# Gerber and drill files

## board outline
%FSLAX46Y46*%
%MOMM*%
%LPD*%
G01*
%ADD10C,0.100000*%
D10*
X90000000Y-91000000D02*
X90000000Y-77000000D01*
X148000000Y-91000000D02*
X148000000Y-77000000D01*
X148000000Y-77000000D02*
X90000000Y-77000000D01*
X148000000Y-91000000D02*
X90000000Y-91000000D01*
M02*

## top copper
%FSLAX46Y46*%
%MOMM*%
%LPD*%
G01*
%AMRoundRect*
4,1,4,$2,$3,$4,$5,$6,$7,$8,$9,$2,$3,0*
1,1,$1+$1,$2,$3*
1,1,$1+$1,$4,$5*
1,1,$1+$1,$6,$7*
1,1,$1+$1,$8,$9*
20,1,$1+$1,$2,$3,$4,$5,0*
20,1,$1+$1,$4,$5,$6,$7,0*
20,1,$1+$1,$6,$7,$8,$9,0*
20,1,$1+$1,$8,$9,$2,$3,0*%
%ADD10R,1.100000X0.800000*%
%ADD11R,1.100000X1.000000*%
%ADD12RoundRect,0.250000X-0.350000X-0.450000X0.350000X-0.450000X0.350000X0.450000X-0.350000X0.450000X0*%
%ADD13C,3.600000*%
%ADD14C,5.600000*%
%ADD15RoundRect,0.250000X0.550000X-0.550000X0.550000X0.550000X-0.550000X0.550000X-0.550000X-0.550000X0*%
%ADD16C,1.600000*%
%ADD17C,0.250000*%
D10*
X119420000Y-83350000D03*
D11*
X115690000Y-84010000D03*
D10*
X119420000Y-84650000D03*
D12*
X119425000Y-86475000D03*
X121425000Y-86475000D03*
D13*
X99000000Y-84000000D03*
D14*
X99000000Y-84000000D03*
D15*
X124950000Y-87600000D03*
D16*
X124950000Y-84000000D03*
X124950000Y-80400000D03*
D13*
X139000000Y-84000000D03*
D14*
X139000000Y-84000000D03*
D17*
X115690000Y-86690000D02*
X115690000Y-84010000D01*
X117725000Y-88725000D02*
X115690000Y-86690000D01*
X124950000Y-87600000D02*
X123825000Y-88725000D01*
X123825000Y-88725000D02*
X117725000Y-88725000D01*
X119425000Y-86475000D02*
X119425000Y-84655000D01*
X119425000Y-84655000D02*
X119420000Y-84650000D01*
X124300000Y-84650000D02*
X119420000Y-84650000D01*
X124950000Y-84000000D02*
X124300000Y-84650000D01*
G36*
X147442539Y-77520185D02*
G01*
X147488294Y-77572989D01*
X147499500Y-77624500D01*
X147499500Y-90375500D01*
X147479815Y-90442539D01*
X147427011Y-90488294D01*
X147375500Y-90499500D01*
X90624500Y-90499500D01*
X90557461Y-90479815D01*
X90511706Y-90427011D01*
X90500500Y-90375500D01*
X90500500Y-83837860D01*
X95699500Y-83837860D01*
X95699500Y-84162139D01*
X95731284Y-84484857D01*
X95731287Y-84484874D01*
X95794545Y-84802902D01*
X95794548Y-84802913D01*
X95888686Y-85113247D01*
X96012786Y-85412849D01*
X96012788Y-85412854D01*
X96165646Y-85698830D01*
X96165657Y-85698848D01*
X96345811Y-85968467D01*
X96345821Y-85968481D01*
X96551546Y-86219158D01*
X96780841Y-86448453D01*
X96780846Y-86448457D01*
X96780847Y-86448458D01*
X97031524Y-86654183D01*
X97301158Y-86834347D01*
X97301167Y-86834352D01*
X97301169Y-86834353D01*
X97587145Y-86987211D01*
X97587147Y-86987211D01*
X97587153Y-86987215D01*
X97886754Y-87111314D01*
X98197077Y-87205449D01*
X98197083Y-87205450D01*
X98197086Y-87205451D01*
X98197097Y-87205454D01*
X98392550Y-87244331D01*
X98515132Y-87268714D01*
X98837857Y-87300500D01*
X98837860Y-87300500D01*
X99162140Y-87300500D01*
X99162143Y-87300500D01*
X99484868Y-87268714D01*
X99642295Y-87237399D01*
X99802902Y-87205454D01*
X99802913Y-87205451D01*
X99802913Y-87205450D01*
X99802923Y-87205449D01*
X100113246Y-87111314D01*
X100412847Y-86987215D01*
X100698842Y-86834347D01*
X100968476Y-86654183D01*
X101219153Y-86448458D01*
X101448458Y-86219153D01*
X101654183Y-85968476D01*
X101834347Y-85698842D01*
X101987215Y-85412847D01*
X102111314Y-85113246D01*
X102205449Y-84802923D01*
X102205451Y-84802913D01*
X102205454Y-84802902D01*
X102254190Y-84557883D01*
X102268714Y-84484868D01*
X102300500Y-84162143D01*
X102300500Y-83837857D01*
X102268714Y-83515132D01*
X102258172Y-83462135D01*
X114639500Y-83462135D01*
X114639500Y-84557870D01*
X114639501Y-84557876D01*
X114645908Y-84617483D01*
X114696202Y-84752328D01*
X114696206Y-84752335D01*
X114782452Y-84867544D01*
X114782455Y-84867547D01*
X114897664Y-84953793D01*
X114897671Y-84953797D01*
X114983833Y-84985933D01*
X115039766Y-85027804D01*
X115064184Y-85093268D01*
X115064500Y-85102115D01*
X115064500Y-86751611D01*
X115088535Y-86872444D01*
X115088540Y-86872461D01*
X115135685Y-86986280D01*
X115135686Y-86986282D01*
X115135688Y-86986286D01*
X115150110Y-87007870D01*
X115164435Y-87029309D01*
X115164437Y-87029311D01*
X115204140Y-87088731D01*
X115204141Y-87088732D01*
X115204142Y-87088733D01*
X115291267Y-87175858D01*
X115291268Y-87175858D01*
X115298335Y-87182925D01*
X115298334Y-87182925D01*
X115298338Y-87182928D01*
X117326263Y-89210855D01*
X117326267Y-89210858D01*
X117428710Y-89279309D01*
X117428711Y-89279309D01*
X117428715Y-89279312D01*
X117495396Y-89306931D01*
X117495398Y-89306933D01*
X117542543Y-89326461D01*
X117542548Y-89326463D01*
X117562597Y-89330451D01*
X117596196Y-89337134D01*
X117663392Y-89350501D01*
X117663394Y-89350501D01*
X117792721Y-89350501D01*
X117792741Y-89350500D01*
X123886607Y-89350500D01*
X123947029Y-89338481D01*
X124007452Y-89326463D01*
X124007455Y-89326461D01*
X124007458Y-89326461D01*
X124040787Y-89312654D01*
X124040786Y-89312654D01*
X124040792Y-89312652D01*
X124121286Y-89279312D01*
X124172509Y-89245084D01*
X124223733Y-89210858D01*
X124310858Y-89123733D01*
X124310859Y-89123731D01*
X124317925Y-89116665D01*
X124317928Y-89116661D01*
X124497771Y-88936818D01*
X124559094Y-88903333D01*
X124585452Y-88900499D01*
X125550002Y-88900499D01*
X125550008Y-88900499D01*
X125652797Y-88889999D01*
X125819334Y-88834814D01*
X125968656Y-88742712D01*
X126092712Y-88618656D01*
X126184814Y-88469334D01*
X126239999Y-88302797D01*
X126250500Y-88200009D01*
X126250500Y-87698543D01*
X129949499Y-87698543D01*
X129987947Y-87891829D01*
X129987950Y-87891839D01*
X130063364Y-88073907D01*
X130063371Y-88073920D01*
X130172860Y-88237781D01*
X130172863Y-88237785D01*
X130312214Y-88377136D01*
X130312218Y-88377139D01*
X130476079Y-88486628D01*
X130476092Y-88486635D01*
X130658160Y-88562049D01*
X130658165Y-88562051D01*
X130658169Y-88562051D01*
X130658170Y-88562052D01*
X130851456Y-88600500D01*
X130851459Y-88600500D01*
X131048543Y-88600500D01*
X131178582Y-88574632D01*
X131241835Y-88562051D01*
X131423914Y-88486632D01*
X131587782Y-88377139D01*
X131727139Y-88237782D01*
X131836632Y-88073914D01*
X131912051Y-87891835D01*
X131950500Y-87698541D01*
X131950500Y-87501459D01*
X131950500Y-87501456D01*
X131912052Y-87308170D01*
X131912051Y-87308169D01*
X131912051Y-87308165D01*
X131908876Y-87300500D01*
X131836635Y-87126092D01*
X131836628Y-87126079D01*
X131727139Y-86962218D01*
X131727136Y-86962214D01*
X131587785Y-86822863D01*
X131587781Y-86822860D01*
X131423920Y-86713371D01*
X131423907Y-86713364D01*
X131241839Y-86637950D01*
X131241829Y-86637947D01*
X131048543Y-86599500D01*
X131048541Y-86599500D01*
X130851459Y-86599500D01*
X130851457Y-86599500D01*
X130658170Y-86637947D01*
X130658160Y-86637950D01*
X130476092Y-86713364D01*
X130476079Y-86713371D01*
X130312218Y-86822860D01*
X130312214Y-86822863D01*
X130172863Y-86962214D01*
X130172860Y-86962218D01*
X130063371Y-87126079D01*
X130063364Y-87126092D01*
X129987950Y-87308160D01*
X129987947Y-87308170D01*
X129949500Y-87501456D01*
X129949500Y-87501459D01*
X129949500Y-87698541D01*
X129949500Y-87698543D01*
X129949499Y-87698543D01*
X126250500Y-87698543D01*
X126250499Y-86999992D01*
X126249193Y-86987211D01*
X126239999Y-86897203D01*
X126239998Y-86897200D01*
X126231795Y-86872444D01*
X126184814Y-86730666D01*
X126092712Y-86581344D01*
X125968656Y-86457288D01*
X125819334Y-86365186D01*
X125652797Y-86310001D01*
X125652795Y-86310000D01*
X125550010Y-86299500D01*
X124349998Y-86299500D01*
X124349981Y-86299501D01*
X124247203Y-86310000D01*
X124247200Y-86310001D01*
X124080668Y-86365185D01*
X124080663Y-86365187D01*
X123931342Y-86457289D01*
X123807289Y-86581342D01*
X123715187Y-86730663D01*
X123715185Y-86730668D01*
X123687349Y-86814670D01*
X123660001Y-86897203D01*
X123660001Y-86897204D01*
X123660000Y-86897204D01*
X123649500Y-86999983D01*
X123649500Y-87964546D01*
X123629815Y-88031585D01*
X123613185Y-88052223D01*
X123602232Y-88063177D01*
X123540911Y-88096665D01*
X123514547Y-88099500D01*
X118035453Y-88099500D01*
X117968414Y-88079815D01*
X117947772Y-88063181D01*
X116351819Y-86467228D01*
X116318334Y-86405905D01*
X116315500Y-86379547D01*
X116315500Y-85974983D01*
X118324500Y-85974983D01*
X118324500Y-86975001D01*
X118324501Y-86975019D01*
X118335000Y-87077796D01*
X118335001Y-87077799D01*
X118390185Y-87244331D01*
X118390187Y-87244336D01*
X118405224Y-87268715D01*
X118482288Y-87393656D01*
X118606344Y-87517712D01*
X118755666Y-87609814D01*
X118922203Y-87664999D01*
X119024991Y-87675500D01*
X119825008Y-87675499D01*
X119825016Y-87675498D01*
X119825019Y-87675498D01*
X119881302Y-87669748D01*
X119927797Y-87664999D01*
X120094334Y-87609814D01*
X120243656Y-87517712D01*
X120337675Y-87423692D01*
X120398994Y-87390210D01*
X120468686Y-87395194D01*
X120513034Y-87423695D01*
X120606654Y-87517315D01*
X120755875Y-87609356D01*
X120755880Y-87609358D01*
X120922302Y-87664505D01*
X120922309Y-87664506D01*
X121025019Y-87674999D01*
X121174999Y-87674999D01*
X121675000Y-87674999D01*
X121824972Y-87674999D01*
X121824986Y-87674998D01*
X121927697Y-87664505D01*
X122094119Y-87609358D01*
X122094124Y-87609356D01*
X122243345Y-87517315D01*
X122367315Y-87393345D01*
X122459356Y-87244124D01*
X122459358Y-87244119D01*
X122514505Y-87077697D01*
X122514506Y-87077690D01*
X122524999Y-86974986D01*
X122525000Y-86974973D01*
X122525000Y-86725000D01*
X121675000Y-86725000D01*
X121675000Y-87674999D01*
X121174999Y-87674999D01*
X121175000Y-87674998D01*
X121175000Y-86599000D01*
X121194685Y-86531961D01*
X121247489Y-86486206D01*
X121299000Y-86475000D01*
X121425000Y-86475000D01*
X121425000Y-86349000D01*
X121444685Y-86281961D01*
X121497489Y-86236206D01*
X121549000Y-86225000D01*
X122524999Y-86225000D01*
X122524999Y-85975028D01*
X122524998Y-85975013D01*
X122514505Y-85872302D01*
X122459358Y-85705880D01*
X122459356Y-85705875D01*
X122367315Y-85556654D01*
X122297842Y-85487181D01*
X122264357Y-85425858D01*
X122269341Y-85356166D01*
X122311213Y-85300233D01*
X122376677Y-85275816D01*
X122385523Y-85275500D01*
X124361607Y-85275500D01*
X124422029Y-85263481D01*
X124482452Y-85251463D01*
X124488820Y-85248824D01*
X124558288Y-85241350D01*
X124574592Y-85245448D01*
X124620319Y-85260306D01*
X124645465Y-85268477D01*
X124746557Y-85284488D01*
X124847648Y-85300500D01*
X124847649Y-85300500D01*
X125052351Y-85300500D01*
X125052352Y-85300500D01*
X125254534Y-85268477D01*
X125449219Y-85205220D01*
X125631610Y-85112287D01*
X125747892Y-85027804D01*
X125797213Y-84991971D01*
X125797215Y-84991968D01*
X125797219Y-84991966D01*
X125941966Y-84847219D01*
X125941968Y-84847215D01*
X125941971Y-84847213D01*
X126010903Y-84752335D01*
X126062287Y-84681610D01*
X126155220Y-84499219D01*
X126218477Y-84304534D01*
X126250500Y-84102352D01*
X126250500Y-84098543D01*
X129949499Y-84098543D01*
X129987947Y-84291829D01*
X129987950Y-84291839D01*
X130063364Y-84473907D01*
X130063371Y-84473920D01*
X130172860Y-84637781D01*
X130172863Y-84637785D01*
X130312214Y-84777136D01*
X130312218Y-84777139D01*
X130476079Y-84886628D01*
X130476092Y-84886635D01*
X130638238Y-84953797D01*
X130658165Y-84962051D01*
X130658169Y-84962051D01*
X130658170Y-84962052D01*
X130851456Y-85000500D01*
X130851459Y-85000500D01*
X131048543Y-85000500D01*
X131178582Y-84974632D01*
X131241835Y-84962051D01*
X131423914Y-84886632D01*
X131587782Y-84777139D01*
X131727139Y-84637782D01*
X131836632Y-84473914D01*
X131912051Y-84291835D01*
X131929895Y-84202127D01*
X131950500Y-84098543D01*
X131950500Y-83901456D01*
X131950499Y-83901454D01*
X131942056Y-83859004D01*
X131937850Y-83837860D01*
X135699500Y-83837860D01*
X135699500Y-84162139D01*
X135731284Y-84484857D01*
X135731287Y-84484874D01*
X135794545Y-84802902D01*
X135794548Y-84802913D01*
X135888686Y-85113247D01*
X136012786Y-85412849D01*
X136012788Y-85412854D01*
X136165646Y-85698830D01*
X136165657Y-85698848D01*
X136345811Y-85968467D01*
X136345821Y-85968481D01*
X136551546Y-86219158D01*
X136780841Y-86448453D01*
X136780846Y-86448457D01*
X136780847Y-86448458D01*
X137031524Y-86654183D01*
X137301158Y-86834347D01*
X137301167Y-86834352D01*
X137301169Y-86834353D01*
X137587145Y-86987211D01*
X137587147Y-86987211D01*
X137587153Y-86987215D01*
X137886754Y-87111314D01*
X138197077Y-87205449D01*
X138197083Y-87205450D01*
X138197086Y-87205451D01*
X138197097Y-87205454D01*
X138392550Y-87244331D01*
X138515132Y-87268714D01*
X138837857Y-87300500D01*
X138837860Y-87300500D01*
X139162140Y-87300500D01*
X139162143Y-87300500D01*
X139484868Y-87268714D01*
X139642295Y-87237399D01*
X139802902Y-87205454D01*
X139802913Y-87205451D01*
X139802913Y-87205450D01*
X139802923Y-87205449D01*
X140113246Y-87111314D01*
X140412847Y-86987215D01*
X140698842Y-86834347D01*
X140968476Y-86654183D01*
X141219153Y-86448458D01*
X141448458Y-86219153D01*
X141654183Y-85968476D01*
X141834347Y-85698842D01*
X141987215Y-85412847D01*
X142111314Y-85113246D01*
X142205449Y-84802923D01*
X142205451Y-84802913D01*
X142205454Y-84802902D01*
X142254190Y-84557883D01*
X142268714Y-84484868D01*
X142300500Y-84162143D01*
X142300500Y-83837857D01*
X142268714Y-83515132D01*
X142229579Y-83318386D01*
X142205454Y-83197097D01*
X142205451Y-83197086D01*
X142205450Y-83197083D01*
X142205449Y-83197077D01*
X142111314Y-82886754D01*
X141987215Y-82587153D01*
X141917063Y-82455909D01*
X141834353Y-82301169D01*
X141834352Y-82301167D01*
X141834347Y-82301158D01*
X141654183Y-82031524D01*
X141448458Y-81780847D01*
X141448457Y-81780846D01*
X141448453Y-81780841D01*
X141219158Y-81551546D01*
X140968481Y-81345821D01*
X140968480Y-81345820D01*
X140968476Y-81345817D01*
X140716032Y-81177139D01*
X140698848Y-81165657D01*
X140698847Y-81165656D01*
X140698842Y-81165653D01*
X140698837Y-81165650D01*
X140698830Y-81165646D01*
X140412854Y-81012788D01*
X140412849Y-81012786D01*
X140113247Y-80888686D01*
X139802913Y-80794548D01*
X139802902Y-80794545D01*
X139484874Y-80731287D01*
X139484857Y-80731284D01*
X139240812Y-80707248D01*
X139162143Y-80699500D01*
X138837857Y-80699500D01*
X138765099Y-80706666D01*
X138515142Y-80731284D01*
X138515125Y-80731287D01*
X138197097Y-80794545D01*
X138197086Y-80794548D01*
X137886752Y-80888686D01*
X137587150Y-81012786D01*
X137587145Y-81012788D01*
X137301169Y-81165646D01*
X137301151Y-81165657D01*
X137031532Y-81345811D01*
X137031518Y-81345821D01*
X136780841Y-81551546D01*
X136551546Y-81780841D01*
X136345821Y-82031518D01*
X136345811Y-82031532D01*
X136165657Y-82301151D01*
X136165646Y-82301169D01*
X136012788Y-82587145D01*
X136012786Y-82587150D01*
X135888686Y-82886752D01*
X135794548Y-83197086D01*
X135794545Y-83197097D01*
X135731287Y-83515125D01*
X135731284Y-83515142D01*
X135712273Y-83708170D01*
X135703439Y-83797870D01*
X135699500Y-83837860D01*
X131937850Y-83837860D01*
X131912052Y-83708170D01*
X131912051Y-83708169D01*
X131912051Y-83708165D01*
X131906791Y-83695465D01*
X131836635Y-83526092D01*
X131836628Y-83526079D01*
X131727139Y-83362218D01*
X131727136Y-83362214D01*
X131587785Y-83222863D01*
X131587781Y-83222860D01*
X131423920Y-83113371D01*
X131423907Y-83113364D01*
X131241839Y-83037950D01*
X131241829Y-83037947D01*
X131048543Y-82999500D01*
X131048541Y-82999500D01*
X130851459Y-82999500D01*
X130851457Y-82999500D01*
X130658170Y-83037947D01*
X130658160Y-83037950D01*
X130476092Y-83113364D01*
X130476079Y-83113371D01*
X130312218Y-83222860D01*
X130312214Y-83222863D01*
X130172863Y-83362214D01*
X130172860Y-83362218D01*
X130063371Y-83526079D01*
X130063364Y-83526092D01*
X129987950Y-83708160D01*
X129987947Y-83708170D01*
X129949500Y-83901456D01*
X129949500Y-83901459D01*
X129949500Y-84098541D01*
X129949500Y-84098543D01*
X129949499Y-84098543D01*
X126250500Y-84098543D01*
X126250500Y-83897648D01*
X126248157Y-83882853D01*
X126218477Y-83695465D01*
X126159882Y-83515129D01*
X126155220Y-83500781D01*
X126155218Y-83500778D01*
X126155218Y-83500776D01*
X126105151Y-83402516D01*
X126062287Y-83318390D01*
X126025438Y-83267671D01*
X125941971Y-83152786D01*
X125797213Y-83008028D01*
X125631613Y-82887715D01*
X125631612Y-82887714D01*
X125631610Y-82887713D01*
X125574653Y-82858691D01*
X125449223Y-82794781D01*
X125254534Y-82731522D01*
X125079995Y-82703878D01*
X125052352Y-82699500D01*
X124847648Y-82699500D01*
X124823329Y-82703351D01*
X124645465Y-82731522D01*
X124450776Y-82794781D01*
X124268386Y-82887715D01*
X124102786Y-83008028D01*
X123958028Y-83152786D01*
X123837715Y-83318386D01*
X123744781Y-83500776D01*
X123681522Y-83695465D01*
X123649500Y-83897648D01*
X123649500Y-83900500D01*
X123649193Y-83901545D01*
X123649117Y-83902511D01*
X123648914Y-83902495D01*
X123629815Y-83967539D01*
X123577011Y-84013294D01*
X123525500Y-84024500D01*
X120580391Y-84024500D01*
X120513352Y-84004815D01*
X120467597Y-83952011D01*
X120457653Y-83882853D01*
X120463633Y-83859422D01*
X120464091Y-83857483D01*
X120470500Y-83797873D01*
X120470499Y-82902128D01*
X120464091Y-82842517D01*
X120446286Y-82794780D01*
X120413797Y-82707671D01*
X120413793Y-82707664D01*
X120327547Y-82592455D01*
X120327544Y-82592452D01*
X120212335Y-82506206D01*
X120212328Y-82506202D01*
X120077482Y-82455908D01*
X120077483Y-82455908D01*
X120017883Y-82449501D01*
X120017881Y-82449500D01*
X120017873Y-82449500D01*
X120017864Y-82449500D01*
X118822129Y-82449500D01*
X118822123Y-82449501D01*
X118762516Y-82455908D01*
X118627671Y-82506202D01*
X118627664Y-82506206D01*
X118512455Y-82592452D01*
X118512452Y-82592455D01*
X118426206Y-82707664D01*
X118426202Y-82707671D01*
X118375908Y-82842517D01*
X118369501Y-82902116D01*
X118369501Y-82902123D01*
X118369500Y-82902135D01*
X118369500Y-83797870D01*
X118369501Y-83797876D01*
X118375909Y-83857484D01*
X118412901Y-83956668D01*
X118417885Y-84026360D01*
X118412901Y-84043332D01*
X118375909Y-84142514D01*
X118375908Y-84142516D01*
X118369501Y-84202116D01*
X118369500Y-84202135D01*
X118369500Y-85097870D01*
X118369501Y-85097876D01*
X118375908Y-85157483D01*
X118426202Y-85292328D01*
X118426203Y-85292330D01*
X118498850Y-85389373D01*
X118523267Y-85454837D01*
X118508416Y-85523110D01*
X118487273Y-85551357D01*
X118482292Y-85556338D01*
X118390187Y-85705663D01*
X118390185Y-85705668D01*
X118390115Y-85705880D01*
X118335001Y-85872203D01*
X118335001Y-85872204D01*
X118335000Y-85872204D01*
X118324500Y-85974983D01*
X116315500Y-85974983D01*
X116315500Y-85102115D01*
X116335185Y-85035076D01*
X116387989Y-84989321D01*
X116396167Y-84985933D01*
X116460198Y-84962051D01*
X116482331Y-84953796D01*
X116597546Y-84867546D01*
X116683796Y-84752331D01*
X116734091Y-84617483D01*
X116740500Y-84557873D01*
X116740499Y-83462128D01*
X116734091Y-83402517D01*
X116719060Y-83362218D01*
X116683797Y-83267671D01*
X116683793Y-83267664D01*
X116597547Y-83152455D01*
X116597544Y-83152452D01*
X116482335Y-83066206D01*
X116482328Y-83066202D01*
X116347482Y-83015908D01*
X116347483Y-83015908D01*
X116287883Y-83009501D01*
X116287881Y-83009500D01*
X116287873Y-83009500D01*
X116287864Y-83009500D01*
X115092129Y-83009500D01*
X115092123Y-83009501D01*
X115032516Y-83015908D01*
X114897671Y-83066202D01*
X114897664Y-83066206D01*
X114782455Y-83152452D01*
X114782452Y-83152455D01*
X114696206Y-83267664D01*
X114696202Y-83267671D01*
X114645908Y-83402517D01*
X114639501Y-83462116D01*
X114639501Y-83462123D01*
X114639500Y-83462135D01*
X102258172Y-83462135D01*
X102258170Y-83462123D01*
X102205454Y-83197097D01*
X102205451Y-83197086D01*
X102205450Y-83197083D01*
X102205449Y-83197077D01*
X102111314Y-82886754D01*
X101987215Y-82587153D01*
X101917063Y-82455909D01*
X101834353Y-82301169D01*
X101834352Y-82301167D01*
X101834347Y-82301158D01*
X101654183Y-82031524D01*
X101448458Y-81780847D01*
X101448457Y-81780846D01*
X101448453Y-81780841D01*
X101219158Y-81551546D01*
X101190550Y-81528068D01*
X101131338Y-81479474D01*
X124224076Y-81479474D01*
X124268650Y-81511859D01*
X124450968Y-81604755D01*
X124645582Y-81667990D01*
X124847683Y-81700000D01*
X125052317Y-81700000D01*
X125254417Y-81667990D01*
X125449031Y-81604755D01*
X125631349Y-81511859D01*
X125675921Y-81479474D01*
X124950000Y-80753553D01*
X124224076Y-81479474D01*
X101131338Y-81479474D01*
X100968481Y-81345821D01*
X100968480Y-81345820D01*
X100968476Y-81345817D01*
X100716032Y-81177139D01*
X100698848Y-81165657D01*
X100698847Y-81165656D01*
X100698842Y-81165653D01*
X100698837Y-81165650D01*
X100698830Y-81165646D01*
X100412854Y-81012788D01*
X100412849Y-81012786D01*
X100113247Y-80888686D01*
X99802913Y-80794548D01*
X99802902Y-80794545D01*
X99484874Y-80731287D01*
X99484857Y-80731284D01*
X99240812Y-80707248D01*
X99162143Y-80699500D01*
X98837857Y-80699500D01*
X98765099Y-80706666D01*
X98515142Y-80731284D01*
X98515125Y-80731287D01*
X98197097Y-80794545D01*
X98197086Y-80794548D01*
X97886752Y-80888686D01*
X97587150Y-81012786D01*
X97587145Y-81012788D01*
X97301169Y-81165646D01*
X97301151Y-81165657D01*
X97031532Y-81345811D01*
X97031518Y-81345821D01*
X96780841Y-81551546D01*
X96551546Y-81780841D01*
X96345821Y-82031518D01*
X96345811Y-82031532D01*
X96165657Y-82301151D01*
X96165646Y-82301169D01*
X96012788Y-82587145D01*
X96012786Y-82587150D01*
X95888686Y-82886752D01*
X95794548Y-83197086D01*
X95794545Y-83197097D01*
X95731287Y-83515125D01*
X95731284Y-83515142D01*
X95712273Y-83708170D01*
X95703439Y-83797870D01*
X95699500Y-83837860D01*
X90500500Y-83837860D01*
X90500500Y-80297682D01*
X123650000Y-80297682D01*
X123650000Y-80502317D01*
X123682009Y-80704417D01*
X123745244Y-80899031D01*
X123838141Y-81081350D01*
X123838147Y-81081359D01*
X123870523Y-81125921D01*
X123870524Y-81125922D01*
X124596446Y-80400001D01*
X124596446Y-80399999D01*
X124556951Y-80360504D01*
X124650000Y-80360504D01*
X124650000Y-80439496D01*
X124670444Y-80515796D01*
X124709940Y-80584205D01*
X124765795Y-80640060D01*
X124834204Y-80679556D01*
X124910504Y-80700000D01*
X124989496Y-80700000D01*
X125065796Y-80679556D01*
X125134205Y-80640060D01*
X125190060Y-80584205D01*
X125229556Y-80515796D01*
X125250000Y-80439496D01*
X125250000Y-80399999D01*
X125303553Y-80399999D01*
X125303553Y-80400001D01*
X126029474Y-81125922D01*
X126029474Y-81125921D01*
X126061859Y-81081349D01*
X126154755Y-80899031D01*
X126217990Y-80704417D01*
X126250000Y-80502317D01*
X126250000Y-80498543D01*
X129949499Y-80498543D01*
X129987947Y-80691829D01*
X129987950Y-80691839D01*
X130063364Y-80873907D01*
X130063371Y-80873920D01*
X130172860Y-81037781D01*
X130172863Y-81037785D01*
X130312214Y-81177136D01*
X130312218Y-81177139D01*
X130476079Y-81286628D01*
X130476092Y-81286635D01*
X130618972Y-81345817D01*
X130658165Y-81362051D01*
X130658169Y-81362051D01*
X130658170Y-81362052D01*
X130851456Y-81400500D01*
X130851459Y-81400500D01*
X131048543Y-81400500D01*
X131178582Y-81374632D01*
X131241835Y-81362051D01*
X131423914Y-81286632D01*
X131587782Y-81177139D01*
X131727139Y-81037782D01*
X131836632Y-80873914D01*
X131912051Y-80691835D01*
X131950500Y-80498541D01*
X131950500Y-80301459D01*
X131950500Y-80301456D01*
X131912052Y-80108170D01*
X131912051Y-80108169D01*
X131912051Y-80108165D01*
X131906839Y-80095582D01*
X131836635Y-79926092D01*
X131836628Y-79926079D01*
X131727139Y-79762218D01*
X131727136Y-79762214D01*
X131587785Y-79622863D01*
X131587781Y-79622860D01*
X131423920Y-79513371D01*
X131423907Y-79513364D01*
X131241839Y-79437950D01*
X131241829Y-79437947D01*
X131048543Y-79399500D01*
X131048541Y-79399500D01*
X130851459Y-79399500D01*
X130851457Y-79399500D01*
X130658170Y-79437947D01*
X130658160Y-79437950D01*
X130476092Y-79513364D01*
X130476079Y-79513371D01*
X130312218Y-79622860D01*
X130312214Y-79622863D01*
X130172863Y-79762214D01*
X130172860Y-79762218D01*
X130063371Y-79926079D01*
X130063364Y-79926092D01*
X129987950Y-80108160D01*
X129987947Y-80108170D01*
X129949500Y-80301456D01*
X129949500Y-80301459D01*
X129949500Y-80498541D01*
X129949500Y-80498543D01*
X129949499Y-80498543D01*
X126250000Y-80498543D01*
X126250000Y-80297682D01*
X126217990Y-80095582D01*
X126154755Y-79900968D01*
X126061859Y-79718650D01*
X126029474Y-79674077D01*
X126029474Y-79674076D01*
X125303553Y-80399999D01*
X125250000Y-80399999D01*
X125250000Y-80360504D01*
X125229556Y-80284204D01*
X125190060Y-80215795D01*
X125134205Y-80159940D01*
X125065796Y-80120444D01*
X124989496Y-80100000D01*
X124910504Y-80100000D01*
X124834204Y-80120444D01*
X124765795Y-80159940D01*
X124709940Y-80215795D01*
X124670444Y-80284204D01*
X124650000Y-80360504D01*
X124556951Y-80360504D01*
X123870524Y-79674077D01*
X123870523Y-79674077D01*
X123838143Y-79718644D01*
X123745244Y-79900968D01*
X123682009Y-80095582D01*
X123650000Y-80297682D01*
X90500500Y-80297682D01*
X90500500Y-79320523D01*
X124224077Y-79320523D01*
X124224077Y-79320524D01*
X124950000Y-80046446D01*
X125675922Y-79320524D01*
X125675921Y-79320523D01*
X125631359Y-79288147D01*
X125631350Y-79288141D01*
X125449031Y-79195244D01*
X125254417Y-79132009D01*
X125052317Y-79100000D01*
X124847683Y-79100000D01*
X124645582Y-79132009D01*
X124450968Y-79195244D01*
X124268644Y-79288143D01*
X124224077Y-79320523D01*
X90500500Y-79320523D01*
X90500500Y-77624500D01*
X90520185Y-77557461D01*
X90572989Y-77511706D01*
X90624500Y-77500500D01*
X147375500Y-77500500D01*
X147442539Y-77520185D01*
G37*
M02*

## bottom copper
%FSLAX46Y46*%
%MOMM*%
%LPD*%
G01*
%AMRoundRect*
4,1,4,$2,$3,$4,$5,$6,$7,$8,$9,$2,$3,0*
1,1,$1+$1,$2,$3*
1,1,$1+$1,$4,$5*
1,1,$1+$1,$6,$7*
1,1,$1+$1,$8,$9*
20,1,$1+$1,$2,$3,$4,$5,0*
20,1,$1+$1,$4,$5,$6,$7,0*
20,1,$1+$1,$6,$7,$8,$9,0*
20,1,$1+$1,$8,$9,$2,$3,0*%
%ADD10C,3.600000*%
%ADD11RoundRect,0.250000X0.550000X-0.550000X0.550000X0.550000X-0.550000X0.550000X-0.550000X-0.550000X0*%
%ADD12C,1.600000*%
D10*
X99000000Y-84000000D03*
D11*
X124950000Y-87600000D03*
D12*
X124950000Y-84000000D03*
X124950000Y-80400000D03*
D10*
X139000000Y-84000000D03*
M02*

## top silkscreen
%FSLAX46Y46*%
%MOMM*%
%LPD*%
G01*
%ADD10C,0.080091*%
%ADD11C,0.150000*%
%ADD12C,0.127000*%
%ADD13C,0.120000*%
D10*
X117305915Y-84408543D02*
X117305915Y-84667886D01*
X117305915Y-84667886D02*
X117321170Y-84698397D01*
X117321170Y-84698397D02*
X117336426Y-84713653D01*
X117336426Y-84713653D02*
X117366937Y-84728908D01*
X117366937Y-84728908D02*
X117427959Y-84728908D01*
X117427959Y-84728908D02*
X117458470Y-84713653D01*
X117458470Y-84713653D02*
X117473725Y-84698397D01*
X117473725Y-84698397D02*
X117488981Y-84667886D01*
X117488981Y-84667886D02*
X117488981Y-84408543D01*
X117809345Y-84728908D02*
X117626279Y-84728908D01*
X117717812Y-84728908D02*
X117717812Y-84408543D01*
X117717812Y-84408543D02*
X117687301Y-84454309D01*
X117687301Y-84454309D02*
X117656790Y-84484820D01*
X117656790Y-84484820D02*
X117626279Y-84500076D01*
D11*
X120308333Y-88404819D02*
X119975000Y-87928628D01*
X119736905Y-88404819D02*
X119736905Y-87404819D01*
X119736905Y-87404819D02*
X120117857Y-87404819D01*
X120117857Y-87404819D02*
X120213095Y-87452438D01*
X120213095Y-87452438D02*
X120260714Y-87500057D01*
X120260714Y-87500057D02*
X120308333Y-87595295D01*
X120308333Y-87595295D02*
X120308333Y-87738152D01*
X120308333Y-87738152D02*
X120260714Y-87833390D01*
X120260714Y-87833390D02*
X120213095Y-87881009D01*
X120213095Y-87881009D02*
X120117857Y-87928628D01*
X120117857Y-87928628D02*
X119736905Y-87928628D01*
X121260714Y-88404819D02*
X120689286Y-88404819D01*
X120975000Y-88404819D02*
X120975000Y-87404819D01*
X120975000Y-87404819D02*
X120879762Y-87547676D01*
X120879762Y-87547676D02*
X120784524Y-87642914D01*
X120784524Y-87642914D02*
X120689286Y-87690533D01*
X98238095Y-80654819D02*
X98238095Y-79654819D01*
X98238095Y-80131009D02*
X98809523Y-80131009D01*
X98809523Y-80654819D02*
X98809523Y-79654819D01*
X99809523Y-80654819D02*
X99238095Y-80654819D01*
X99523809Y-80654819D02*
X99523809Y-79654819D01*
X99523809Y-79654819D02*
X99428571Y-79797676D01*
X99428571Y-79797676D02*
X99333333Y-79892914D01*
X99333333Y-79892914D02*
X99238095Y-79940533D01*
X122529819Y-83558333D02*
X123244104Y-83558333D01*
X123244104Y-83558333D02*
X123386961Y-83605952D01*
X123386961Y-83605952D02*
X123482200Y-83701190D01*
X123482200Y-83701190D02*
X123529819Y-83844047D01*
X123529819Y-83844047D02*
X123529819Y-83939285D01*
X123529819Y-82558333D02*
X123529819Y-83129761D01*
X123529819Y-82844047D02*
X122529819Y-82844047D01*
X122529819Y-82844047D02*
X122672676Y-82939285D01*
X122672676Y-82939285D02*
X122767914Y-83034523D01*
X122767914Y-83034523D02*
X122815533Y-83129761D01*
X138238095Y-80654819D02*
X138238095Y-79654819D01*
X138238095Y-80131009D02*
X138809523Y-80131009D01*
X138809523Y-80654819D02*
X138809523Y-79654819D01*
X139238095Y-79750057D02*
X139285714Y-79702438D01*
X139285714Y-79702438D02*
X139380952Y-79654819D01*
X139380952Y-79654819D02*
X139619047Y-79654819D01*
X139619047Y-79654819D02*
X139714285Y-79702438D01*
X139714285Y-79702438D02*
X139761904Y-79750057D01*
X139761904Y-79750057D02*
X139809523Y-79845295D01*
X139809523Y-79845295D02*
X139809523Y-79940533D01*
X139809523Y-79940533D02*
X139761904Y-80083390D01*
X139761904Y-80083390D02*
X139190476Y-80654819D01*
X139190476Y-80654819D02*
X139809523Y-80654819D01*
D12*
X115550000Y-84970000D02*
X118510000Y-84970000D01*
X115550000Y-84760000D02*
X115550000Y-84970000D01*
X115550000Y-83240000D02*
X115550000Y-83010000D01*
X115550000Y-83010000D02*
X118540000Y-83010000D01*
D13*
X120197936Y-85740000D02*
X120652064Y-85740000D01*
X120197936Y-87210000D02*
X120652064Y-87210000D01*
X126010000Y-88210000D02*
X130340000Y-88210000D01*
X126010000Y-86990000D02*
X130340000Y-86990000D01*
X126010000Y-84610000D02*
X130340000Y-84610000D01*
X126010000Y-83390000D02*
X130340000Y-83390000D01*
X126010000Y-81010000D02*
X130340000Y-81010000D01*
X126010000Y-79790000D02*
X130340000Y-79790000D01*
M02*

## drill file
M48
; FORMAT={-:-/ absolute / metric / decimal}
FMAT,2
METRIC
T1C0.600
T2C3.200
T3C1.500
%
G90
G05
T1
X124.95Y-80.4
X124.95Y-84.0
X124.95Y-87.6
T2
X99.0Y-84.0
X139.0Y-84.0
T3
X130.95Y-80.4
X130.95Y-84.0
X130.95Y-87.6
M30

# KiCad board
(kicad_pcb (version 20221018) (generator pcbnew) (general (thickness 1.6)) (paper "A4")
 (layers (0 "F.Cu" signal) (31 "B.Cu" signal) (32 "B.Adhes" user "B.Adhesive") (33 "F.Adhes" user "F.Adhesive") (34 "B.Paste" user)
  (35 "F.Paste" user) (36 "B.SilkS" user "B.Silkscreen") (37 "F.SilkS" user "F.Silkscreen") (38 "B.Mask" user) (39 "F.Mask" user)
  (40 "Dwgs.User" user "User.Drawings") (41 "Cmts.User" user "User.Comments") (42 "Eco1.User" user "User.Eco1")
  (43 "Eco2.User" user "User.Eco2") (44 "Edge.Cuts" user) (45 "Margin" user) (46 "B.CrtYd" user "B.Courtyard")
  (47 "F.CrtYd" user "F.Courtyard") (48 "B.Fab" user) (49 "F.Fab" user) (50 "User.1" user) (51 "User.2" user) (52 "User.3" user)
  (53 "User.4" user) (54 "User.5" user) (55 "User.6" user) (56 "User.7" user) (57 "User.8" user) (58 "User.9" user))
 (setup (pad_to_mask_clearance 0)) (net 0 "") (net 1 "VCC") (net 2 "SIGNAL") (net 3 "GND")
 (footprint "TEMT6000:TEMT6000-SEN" (layer "F.Cu") (at 117.55 84 180)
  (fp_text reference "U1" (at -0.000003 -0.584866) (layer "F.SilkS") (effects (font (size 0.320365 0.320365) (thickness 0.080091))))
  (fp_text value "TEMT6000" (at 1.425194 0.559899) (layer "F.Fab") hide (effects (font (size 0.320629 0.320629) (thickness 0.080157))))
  (fp_line (start 2 -0.97) (end -0.96 -0.97) (stroke (width 0.127) (type solid)) (layer "F.SilkS"))
  (fp_line (start 2 -0.76) (end 2 -0.97) (stroke (width 0.127) (type solid)) (layer "F.SilkS"))
  (fp_line (start 2 0.76) (end 2 0.99) (stroke (width 0.127) (type solid)) (layer "F.SilkS"))
  (fp_line (start 2 0.99) (end -0.99 0.99) (stroke (width 0.127) (type solid)) (layer "F.SilkS"))
  (pad "BASE" smd rect (at -1.87 0.65 180) (size 1.1 0.8) (layers "F.Cu" "F.Paste" "F.Mask"))
  (pad "COLLECTOR" smd rect (at 1.86 -0.01 180) (size 1.1 1) (layers "F.Cu" "F.Paste" "F.Mask") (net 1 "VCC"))
  (pad "EMITTER" smd rect (at -1.87 -0.65 180) (size 1.1 0.8) (layers "F.Cu" "F.Paste" "F.Mask") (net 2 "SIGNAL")))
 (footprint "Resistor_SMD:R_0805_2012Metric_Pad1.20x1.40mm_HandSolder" (layer "F.Cu") (at 120.425 86.475)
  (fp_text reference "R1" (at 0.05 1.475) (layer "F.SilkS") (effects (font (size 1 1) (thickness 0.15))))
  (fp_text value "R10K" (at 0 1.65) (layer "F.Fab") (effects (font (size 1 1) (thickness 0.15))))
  (fp_line (start -0.227064 -0.735) (end 0.227064 -0.735) (stroke (width 0.12) (type solid)) (layer "F.SilkS"))
  (fp_line (start -0.227064 0.735) (end 0.227064 0.735) (stroke (width 0.12) (type solid)) (layer "F.SilkS"))
  (pad "1" smd roundrect (at -1 0) (size 1.2 1.4) (layers "F.Cu" "F.Paste" "F.Mask") (roundrect_rratio 0.2083333333) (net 2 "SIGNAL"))
  (pad "2" smd roundrect (at 1 0) (size 1.2 1.4) (layers "F.Cu" "F.Paste" "F.Mask") (roundrect_rratio 0.2083333333) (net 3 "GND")))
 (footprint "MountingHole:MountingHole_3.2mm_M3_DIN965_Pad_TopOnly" (layer "F.Cu") (at 99 84)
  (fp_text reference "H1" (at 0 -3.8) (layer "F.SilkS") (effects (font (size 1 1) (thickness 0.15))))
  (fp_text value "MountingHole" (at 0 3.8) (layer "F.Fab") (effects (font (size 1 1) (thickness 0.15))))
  (pad "1" thru_hole circle (at 0 0) (size 3.6 3.6) (drill 3.2) (layers "*.Cu" "*.Mask"))
  (pad "1" connect circle (at 0 0) (size 5.6 5.6) (layers "F.Cu" "F.Mask")))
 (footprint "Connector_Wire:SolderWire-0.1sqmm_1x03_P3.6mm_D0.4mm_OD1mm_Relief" (layer "F.Cu") (at 124.95 87.6 90)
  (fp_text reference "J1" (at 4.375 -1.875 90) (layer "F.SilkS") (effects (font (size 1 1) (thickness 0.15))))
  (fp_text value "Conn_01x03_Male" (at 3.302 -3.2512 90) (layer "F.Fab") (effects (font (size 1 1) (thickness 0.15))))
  (fp_line (start -0.61 1.06) (end -0.61 5.39) (stroke (width 0.12) (type solid)) (layer "F.SilkS"))
  (fp_line (start 0.61 1.06) (end 0.61 5.39) (stroke (width 0.12) (type solid)) (layer "F.SilkS"))
  (fp_line (start 2.99 1.06) (end 2.99 5.39) (stroke (width 0.12) (type solid)) (layer "F.SilkS"))
  (fp_line (start 4.21 1.06) (end 4.21 5.39) (stroke (width 0.12) (type solid)) (layer "F.SilkS"))
  (fp_line (start 6.59 1.06) (end 6.59 5.39) (stroke (width 0.12) (type solid)) (layer "F.SilkS"))
  (fp_line (start 7.81 1.06) (end 7.81 5.39) (stroke (width 0.12) (type solid)) (layer "F.SilkS"))
  (pad "" np_thru_hole circle (at 0 6 90) (size 1.5 1.5) (drill 1.5) (layers "*.Cu" "*.Mask"))
  (pad "" np_thru_hole circle (at 3.6 6 90) (size 1.5 1.5) (drill 1.5) (layers "*.Cu" "*.Mask"))
  (pad "" np_thru_hole circle (at 7.2 6 90) (size 1.5 1.5) (drill 1.5) (layers "*.Cu" "*.Mask"))
  (pad "1" thru_hole roundrect (at 0 0 90) (size 1.6 1.6) (drill 0.6) (layers "*.Cu" "*.Mask") (roundrect_rratio 0.15625) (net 1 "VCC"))
  (pad "2" thru_hole circle (at 3.6 0 90) (size 1.6 1.6) (drill 0.6) (layers "*.Cu" "*.Mask") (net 2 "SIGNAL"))
  (pad "3" thru_hole circle (at 7.2 0 90) (size 1.6 1.6) (drill 0.6) (layers "*.Cu" "*.Mask") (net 3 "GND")))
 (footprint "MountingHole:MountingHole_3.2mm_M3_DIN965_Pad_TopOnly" (layer "F.Cu") (at 139 84)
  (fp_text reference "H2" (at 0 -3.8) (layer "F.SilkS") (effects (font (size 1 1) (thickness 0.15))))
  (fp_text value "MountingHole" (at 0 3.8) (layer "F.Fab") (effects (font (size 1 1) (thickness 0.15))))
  (pad "1" thru_hole circle (at 0 0) (size 3.6 3.6) (drill 3.2) (layers "*.Cu" "*.Mask"))
  (pad "1" connect circle (at 0 0) (size 5.6 5.6) (layers "F.Cu" "F.Mask")))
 (gr_line (start 90 91) (end 90 77) (stroke (width 0.1) (type default)) (layer "Edge.Cuts"))
 (gr_line (start 148 91) (end 148 77) (stroke (width 0.1) (type default)) (layer "Edge.Cuts"))
 (gr_line (start 148 77) (end 90 77) (stroke (width 0.1) (type default)) (layer "Edge.Cuts"))
 (gr_line (start 148 91) (end 90 91) (stroke (width 0.1) (type default)) (layer "Edge.Cuts"))
 (segment (start 115.69 86.69) (end 115.69 84.01) (width 0.25) (layer "F.Cu") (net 1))
 (segment (start 117.725 88.725) (end 115.69 86.69) (width 0.25) (layer "F.Cu") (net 1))
 (segment (start 124.95 87.6) (end 123.825 88.725) (width 0.25) (layer "F.Cu") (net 1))
 (segment (start 123.825 88.725) (end 117.725 88.725) (width 0.25) (layer "F.Cu") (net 1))
 (segment (start 119.425 86.475) (end 119.425 84.655) (width 0.25) (layer "F.Cu") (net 2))
 (segment (start 119.425 84.655) (end 119.42 84.65) (width 0.25) (layer "F.Cu") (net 2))
 (segment (start 124.3 84.65) (end 119.42 84.65) (width 0.25) (layer "F.Cu") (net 2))
 (segment (start 124.95 84) (end 124.3 84.65) (width 0.25) (layer "F.Cu") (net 2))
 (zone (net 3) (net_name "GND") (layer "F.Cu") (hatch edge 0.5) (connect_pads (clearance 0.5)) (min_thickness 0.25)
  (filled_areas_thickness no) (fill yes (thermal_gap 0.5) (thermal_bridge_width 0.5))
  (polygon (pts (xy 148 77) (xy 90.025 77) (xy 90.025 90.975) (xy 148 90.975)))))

